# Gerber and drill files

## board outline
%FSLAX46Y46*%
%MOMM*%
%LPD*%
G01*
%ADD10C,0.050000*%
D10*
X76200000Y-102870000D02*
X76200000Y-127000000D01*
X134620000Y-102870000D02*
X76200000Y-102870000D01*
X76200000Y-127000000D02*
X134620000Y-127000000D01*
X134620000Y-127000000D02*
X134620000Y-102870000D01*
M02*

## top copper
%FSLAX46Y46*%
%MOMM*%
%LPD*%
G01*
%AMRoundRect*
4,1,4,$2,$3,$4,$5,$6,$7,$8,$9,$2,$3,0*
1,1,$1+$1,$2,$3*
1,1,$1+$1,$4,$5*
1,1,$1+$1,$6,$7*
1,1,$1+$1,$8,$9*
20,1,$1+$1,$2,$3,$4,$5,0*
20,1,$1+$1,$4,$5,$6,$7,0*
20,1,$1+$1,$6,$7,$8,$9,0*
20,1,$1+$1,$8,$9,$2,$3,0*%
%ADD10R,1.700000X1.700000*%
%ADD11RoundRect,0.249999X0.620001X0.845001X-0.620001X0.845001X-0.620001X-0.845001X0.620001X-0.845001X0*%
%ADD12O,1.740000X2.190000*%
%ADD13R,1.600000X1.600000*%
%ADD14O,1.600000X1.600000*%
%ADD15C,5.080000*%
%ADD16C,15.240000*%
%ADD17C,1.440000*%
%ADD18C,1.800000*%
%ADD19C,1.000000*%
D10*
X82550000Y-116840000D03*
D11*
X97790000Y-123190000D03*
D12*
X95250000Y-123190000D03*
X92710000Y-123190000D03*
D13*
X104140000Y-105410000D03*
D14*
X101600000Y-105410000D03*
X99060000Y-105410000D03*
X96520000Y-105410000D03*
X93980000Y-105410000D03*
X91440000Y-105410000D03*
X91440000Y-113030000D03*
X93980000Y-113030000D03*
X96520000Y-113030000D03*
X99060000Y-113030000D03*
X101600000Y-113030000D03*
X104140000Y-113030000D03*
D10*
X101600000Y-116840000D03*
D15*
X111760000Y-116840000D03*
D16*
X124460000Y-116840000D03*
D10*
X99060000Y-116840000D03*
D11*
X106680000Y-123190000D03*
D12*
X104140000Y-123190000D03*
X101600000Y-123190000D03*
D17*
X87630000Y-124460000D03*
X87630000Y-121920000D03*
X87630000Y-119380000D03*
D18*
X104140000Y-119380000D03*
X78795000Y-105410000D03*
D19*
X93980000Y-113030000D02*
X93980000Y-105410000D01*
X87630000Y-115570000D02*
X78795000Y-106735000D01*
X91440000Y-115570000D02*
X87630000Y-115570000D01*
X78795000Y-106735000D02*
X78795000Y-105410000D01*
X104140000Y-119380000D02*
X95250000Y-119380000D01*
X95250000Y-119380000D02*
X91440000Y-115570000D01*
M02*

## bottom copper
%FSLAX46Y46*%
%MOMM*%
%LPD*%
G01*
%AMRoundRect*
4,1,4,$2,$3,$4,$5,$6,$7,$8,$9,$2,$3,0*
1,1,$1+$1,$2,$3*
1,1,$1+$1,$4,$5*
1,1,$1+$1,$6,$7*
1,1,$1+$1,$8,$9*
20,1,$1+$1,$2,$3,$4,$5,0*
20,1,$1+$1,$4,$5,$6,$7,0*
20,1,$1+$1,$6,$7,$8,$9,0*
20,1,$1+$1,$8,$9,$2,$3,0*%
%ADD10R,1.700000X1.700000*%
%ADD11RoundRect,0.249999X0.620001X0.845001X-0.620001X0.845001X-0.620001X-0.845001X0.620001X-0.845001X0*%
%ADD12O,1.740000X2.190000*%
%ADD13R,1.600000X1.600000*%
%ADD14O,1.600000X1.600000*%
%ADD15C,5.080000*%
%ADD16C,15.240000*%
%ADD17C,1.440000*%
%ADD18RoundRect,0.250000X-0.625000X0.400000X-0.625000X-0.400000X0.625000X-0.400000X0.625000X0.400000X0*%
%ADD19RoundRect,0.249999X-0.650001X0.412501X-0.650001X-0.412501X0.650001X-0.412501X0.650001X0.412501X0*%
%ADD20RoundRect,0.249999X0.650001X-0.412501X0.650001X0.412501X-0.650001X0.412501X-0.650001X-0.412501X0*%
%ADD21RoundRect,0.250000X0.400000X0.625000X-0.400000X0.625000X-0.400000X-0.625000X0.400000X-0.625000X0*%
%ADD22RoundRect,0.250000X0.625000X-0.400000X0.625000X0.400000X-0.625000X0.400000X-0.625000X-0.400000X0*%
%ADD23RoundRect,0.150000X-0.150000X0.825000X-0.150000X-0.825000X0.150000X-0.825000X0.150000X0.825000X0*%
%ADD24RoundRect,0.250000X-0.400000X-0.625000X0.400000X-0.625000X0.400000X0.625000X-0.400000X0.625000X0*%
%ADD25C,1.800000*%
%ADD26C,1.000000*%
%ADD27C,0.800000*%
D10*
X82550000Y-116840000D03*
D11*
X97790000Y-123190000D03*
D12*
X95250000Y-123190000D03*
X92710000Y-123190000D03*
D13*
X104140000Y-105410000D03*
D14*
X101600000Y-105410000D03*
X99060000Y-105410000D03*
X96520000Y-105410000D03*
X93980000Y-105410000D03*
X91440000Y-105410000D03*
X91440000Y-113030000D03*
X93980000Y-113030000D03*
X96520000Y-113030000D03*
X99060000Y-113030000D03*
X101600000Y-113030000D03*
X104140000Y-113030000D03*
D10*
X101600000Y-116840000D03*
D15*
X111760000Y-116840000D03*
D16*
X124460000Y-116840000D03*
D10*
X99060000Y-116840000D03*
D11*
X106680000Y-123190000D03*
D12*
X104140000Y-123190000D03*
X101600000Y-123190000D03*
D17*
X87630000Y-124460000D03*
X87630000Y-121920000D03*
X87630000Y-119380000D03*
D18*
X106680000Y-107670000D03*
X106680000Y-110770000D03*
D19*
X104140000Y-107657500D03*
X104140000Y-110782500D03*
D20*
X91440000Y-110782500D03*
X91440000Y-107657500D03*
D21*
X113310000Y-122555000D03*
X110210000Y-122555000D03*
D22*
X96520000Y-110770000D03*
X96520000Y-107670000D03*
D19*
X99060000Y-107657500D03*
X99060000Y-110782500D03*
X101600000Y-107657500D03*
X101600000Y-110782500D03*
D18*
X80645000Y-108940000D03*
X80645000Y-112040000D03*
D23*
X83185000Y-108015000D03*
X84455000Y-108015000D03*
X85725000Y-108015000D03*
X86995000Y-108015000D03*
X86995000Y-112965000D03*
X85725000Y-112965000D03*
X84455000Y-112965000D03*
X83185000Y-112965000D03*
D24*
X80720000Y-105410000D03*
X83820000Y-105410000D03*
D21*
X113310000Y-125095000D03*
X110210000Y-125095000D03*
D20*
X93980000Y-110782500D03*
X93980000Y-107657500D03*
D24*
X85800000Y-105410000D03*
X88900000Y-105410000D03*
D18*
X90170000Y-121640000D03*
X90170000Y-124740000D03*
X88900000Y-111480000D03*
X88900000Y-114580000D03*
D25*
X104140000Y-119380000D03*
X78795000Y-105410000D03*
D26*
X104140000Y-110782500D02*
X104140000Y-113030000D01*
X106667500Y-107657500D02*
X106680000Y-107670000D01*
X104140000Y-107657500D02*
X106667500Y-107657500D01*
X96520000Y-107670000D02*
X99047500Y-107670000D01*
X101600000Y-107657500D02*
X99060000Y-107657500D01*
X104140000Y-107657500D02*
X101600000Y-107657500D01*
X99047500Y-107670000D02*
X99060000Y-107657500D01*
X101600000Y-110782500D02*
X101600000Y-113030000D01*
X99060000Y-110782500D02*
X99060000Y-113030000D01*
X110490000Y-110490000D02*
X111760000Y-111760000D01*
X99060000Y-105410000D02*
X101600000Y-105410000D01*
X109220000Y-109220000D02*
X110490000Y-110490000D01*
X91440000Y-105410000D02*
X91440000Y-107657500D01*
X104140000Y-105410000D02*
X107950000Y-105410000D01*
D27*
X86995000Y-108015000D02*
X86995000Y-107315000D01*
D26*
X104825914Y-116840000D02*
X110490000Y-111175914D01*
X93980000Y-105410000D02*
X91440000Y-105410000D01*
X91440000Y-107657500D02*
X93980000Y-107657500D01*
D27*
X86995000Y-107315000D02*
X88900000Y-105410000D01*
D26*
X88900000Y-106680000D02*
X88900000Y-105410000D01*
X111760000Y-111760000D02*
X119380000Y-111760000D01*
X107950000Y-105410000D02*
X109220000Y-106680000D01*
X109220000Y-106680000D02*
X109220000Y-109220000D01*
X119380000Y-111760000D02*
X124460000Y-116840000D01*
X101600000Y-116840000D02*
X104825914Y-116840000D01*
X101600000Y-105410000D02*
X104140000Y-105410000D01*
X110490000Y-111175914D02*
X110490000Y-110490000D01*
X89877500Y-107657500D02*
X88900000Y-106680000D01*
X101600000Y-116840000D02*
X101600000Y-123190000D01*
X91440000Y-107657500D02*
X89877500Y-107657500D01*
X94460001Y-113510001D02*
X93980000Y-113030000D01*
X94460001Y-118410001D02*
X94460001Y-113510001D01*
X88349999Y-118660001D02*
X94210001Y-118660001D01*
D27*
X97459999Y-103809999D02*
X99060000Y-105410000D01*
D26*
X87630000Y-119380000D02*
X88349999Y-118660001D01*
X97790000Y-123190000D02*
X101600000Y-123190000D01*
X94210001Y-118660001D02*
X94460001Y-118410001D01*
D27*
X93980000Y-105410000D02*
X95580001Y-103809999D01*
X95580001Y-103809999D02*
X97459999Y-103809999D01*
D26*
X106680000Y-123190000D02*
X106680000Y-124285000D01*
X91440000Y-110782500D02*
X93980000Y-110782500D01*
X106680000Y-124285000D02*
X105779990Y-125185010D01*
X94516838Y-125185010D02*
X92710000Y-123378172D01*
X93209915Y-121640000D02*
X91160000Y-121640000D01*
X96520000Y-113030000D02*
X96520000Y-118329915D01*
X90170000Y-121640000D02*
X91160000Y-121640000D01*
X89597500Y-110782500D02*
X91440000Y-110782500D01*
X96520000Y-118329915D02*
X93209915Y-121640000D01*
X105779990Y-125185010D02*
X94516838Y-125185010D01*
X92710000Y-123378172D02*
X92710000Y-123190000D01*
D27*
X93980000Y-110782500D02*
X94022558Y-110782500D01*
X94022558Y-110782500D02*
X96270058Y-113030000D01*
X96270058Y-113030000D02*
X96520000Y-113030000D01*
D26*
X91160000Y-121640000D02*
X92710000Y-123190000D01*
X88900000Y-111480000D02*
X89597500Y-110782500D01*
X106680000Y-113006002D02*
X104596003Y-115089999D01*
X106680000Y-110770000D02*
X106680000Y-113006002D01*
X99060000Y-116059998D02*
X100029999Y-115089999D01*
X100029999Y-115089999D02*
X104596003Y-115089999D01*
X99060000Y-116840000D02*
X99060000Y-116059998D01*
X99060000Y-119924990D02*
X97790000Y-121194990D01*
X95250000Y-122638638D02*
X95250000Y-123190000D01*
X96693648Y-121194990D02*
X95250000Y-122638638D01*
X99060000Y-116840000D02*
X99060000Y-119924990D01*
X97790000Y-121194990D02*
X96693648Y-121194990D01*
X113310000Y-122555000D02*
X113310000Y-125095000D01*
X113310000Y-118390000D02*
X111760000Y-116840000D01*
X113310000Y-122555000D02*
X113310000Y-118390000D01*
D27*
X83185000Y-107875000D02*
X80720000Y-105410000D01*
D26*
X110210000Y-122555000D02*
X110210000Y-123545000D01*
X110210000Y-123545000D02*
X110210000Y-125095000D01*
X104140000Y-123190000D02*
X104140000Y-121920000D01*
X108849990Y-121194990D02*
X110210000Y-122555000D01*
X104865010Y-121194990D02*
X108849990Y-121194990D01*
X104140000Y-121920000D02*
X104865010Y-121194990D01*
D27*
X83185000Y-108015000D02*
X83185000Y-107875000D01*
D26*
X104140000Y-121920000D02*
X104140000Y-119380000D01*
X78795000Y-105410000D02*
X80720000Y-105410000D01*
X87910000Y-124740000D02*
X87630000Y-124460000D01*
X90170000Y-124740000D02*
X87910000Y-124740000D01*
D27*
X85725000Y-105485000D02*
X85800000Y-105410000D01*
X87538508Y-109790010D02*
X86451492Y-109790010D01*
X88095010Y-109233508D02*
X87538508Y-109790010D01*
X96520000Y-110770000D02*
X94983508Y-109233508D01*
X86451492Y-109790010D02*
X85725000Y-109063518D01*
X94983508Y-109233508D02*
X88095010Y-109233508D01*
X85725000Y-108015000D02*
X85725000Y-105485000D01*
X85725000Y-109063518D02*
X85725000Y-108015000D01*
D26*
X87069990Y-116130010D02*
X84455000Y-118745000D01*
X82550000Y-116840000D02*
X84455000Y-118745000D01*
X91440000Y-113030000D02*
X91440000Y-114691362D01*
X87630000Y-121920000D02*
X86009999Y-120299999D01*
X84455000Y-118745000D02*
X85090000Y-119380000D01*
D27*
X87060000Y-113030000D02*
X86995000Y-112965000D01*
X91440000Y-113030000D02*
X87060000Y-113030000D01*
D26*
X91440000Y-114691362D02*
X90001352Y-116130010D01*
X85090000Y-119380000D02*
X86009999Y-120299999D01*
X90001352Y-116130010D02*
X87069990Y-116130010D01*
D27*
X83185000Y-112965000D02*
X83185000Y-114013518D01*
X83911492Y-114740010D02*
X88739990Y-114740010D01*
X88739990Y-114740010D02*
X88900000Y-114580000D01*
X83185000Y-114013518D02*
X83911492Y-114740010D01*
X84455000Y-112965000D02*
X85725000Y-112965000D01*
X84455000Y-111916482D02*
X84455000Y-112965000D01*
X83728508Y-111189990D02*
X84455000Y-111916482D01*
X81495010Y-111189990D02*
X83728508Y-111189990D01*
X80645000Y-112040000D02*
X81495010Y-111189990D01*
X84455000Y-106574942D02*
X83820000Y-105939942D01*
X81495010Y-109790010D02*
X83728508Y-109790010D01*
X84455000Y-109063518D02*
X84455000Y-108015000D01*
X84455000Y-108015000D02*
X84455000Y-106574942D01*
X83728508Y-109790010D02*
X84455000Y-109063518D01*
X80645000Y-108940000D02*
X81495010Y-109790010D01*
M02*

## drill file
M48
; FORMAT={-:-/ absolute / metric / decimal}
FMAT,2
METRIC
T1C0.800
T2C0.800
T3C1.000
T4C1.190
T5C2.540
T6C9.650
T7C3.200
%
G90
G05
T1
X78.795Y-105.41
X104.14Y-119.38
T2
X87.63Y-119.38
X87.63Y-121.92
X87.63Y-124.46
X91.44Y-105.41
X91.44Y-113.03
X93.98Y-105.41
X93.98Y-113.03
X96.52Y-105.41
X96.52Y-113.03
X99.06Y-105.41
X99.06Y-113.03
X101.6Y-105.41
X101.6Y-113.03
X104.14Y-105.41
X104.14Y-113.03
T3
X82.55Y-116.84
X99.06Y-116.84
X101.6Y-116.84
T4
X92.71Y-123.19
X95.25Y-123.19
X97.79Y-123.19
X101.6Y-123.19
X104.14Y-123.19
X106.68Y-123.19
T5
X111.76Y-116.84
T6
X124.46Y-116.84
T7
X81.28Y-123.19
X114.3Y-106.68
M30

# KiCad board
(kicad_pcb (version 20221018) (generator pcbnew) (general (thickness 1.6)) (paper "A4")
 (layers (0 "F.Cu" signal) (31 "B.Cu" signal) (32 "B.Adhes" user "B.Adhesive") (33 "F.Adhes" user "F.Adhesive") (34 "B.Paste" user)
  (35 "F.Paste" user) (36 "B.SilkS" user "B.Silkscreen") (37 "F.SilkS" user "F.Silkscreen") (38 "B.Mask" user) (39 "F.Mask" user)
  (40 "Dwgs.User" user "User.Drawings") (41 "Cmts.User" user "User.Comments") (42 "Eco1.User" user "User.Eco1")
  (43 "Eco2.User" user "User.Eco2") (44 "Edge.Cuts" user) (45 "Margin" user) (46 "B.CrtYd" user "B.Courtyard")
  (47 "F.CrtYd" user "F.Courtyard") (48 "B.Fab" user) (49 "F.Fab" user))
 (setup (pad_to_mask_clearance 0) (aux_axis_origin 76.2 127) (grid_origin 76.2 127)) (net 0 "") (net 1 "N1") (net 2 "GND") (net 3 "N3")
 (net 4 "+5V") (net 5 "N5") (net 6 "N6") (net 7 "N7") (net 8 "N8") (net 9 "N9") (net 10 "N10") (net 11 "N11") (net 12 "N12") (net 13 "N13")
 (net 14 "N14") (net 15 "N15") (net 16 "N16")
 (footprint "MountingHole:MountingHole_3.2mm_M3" (layer "F.Cu") (at 114.3 106.68)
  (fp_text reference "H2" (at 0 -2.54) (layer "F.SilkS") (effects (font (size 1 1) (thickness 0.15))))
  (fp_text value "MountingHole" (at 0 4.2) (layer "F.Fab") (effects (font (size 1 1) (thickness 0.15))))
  (pad "" np_thru_hole circle (at 0 0) (size 3.2 3.2) (drill 3.2) (layers "*.Cu" "*.Mask")))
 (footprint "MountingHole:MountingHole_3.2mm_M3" (layer "F.Cu") (at 81.28 123.19)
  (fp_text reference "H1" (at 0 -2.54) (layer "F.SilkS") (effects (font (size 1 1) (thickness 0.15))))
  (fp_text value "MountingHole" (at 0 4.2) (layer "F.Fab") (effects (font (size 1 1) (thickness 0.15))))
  (pad "" np_thru_hole circle (at 0 0) (size 3.2 3.2) (drill 3.2) (layers "*.Cu" "*.Mask")))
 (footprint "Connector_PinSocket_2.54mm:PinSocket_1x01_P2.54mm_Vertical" (layer "F.Cu") (at 82.55 116.84)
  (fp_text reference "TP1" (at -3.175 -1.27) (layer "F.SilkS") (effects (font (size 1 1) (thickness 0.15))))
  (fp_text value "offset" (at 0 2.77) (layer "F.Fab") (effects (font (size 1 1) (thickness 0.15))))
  (pad "1" thru_hole rect (at 0 0) (size 1.7 1.7) (drill 1) (layers "*.Cu" "*.Mask") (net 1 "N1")))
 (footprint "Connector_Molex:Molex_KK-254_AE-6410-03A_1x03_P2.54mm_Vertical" (layer "F.Cu") (at 97.79 123.19 180)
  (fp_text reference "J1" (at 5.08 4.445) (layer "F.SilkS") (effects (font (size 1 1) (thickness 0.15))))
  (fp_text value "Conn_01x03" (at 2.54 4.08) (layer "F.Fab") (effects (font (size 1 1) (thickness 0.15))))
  (pad "1" thru_hole roundrect (at 0 0 180) (size 1.74 2.19) (drill 1.19) (layers "*.Cu" "*.Mask") (roundrect_rratio 0.1436775862)
   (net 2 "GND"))
  (pad "2" thru_hole oval (at 2.54 0 180) (size 1.74 2.19) (drill 1.19) (layers "*.Cu" "*.Mask") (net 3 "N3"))
  (pad "3" thru_hole oval (at 5.08 0 180) (size 1.74 2.19) (drill 1.19) (layers "*.Cu" "*.Mask") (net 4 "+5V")))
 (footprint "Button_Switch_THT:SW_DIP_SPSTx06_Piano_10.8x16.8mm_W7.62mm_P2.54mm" (layer "F.Cu") (at 104.14 105.41 -90)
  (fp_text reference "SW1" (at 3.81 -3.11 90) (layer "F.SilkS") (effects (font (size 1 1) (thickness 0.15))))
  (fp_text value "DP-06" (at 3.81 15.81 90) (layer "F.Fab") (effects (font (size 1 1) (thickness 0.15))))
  (pad "1" thru_hole rect (at 0 0 270) (size 1.6 1.6) (drill 0.8) (layers "*.Cu" "*.Mask") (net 2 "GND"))
  (pad "2" thru_hole oval (at 0 2.54 270) (size 1.6 1.6) (drill 0.8) (layers "*.Cu" "*.Mask") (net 2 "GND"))
  (pad "3" thru_hole oval (at 0 5.08 270) (size 1.6 1.6) (drill 0.8) (layers "*.Cu" "*.Mask") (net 2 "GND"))
  (pad "4" thru_hole oval (at 0 7.62 270) (size 1.6 1.6) (drill 0.8) (layers "*.Cu" "*.Mask") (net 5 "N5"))
  (pad "5" thru_hole oval (at 0 10.16 270) (size 1.6 1.6) (drill 0.8) (layers "*.Cu" "*.Mask") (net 2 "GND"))
  (pad "6" thru_hole oval (at 0 12.7 270) (size 1.6 1.6) (drill 0.8) (layers "*.Cu" "*.Mask") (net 2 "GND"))
  (pad "7" thru_hole oval (at 7.62 12.7 270) (size 1.6 1.6) (drill 0.8) (layers "*.Cu" "*.Mask") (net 1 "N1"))
  (pad "8" thru_hole oval (at 7.62 10.16 270) (size 1.6 1.6) (drill 0.8) (layers "*.Cu" "*.Mask") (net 2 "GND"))
  (pad "9" thru_hole oval (at 7.62 7.62 270) (size 1.6 1.6) (drill 0.8) (layers "*.Cu" "*.Mask") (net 4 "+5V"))
  (pad "10" thru_hole oval (at 7.62 5.08 270) (size 1.6 1.6) (drill 0.8) (layers "*.Cu" "*.Mask") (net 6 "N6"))
  (pad "11" thru_hole oval (at 7.62 2.54 270) (size 1.6 1.6) (drill 0.8) (layers "*.Cu" "*.Mask") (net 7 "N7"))
  (pad "12" thru_hole oval (at 7.62 0 270) (size 1.6 1.6) (drill 0.8) (layers "*.Cu" "*.Mask") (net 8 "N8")))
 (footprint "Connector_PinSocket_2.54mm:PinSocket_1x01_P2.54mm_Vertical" (layer "F.Cu") (at 101.6 116.84)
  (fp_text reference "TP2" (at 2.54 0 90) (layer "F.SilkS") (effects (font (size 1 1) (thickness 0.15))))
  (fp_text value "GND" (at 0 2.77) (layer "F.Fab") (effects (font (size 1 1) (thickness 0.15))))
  (pad "1" thru_hole rect (at 0 0) (size 1.7 1.7) (drill 1) (layers "*.Cu" "*.Mask") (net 2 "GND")))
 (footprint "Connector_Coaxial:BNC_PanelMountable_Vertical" (layer "F.Cu") (at 111.76 116.84 180)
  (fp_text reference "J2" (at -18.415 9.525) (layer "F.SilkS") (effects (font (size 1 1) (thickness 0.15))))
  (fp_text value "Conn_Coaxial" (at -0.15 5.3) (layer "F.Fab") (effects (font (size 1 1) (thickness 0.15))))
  (pad "1" thru_hole circle (at 0 0 180) (size 5.08 5.08) (drill 2.54) (layers "*.Cu" "*.Mask") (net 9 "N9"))
  (pad "2" thru_hole circle (at -12.7 0 180) (size 15.24 15.24) (drill 9.65) (layers "*.Cu" "*.Mask") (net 2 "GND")))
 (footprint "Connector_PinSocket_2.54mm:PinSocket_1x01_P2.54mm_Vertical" (layer "F.Cu") (at 99.06 116.84)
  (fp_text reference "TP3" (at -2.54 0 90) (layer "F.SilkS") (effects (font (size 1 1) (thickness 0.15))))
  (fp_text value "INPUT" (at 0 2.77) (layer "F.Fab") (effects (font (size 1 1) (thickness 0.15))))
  (pad "1" thru_hole rect (at 0 0) (size 1.7 1.7) (drill 1) (layers "*.Cu" "*.Mask") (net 3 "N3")))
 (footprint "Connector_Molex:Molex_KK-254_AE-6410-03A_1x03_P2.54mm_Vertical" (layer "F.Cu") (at 106.68 123.19 180)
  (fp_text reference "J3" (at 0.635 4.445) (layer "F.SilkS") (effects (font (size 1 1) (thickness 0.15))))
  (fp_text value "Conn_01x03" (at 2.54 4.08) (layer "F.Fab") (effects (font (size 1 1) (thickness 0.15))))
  (pad "1" thru_hole roundrect (at 0 0 180) (size 1.74 2.19) (drill 1.19) (layers "*.Cu" "*.Mask") (roundrect_rratio 0.1436775862)
   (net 4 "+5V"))
  (pad "2" thru_hole oval (at 2.54 0 180) (size 1.74 2.19) (drill 1.19) (layers "*.Cu" "*.Mask") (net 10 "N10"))
  (pad "3" thru_hole oval (at 5.08 0 180) (size 1.74 2.19) (drill 1.19) (layers "*.Cu" "*.Mask") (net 2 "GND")))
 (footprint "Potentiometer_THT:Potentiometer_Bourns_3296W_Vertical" (layer "F.Cu") (at 87.63 124.46 -90)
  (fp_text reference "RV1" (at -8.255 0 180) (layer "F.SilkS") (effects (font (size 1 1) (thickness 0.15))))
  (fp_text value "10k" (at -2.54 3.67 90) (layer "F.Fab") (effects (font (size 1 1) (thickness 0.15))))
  (pad "1" thru_hole circle (at 0 0 270) (size 1.44 1.44) (drill 0.8) (layers "*.Cu" "*.Mask") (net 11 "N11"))
  (pad "2" thru_hole circle (at -2.54 0 270) (size 1.44 1.44) (drill 0.8) (layers "*.Cu" "*.Mask") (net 1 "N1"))
  (pad "3" thru_hole circle (at -5.08 0 270) (size 1.44 1.44) (drill 0.8) (layers "*.Cu" "*.Mask") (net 2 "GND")))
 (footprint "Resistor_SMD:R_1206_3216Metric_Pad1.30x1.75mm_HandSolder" (layer "B.Cu") (at 106.68 109.22 -90)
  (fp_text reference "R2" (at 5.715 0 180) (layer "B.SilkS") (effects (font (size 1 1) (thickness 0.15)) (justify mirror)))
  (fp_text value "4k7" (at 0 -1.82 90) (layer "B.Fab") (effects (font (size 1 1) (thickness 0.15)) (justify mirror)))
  (pad "1" smd roundrect (at -1.55 0 270) (size 1.3 1.75) (layers "B.Cu" "B.Paste" "B.Mask") (roundrect_rratio 0.1923076923) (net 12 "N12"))
  (pad "2" smd roundrect (at 1.55 0 270) (size 1.3 1.75) (layers "B.Cu" "B.Paste" "B.Mask") (roundrect_rratio 0.1923076923) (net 3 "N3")))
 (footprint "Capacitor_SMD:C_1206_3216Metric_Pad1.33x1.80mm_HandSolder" (layer "B.Cu") (at 104.14 109.22 -90)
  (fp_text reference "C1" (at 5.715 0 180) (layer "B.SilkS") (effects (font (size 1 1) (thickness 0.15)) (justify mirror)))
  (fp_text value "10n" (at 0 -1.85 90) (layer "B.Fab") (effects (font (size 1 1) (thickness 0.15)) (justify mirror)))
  (pad "1" smd roundrect (at -1.5625 0 270) (size 1.325 1.8) (layers "B.Cu" "B.Paste" "B.Mask") (roundrect_rratio 0.1886784906)
   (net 12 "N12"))
  (pad "2" smd roundrect (at 1.5625 0 270) (size 1.325 1.8) (layers "B.Cu" "B.Paste" "B.Mask") (roundrect_rratio 0.1886784906) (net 8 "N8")))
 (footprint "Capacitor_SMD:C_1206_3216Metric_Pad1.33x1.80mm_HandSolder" (layer "B.Cu") (at 91.44 109.22 90)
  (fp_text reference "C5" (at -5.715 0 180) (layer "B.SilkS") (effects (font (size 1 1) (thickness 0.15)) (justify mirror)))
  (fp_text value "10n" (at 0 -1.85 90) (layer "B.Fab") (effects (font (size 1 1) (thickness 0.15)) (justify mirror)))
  (pad "1" smd roundrect (at -1.5625 0 90) (size 1.325 1.8) (layers "B.Cu" "B.Paste" "B.Mask") (roundrect_rratio 0.1886784906) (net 4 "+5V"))
  (pad "2" smd roundrect (at 1.5625 0 90) (size 1.325 1.8) (layers "B.Cu" "B.Paste" "B.Mask") (roundrect_rratio 0.1886784906) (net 2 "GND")))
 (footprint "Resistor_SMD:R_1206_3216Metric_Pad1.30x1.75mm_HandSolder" (layer "B.Cu") (at 111.76 122.555 180)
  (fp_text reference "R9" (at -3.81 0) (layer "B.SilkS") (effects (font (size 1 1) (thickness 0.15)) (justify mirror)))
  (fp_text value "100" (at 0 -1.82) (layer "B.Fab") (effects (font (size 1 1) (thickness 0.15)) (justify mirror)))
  (pad "1" smd roundrect (at -1.55 0 180) (size 1.3 1.75) (layers "B.Cu" "B.Paste" "B.Mask") (roundrect_rratio 0.1923076923) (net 9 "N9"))
  (pad "2" smd roundrect (at 1.55 0 180) (size 1.3 1.75) (layers "B.Cu" "B.Paste" "B.Mask") (roundrect_rratio 0.1923076923) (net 10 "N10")))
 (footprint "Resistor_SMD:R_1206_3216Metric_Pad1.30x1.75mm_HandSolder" (layer "B.Cu") (at 96.52 109.22 90)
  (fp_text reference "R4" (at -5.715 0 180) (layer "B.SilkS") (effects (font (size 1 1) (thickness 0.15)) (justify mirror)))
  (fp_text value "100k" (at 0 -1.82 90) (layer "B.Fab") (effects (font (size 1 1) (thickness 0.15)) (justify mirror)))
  (pad "1" smd roundrect (at -1.55 0 90) (size 1.3 1.75) (layers "B.Cu" "B.Paste" "B.Mask") (roundrect_rratio 0.1923076923) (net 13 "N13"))
  (pad "2" smd roundrect (at 1.55 0 90) (size 1.3 1.75) (layers "B.Cu" "B.Paste" "B.Mask") (roundrect_rratio 0.1923076923) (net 12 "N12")))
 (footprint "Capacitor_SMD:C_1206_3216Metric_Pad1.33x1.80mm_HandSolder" (layer "B.Cu") (at 99.06 109.22 -90)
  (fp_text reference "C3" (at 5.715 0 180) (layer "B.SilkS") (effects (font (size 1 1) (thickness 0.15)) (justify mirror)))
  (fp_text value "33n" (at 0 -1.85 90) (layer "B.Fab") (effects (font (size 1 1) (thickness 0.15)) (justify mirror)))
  (pad "1" smd roundrect (at -1.5625 0 270) (size 1.325 1.8) (layers "B.Cu" "B.Paste" "B.Mask") (roundrect_rratio 0.1886784906)
   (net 12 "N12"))
  (pad "2" smd roundrect (at 1.5625 0 270) (size 1.325 1.8) (layers "B.Cu" "B.Paste" "B.Mask") (roundrect_rratio 0.1886784906) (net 6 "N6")))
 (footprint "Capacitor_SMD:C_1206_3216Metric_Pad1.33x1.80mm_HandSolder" (layer "B.Cu") (at 101.6 109.22 -90)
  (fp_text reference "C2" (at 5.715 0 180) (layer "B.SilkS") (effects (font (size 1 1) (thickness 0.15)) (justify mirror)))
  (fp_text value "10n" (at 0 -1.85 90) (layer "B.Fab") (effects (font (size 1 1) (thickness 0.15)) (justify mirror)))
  (pad "1" smd roundrect (at -1.5625 0 270) (size 1.325 1.8) (layers "B.Cu" "B.Paste" "B.Mask") (roundrect_rratio 0.1886784906)
   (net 12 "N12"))
  (pad "2" smd roundrect (at 1.5625 0 270) (size 1.325 1.8) (layers "B.Cu" "B.Paste" "B.Mask") (roundrect_rratio 0.1886784906) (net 7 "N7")))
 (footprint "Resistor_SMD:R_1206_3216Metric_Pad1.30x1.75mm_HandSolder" (layer "B.Cu") (at 80.645 110.49 -90)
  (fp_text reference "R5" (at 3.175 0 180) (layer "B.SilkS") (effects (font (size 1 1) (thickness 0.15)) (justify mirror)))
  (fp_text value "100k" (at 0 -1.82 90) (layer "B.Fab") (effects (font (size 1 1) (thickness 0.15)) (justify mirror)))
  (pad "1" smd roundrect (at -1.55 0 270) (size 1.3 1.75) (layers "B.Cu" "B.Paste" "B.Mask") (roundrect_rratio 0.1923076923) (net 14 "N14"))
  (pad "2" smd roundrect (at 1.55 0 270) (size 1.3 1.75) (layers "B.Cu" "B.Paste" "B.Mask") (roundrect_rratio 0.1923076923) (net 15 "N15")))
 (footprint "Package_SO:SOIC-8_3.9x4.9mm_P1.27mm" (layer "B.Cu") (at 85.09 110.49 -90)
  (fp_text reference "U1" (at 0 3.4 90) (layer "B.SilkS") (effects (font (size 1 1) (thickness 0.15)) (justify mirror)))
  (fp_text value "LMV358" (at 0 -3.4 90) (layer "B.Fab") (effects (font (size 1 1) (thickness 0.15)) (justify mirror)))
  (pad "1" smd roundrect (at -2.475 1.905 270) (size 1.95 0.6) (layers "B.Cu" "B.Paste" "B.Mask") (roundrect_rratio 0.25) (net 10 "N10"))
  (pad "2" smd roundrect (at -2.475 0.635 270) (size 1.95 0.6) (layers "B.Cu" "B.Paste" "B.Mask") (roundrect_rratio 0.25) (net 14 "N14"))
  (pad "3" smd roundrect (at -2.475 -0.635 270) (size 1.95 0.6) (layers "B.Cu" "B.Paste" "B.Mask") (roundrect_rratio 0.25) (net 13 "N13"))
  (pad "4" smd roundrect (at -2.475 -1.905 270) (size 1.95 0.6) (layers "B.Cu" "B.Paste" "B.Mask") (roundrect_rratio 0.25) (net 2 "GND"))
  (pad "5" smd roundrect (at 2.475 -1.905 270) (size 1.95 0.6) (layers "B.Cu" "B.Paste" "B.Mask") (roundrect_rratio 0.25) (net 1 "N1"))
  (pad "6" smd roundrect (at 2.475 -0.635 270) (size 1.95 0.6) (layers "B.Cu" "B.Paste" "B.Mask") (roundrect_rratio 0.25) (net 15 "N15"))
  (pad "7" smd roundrect (at 2.475 0.635 270) (size 1.95 0.6) (layers "B.Cu" "B.Paste" "B.Mask") (roundrect_rratio 0.25) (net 15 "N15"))
  (pad "8" smd roundrect (at 2.475 1.905 270) (size 1.95 0.6) (layers "B.Cu" "B.Paste" "B.Mask") (roundrect_rratio 0.25) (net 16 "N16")))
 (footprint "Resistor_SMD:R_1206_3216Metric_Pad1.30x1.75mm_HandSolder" (layer "B.Cu") (at 82.27 105.41)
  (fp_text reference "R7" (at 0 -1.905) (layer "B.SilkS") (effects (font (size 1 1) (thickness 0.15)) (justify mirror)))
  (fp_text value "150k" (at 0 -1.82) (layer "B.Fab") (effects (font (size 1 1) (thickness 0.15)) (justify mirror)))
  (pad "1" smd roundrect (at -1.55 0) (size 1.3 1.75) (layers "B.Cu" "B.Paste" "B.Mask") (roundrect_rratio 0.1923076923) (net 10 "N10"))
  (pad "2" smd roundrect (at 1.55 0) (size 1.3 1.75) (layers "B.Cu" "B.Paste" "B.Mask") (roundrect_rratio 0.1923076923) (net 14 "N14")))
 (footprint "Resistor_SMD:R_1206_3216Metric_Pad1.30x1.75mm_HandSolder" (layer "B.Cu") (at 111.76 125.095 180)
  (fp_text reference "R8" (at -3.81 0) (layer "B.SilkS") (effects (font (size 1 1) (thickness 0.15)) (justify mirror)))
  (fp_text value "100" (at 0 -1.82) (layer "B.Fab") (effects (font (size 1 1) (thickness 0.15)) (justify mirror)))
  (pad "1" smd roundrect (at -1.55 0 180) (size 1.3 1.75) (layers "B.Cu" "B.Paste" "B.Mask") (roundrect_rratio 0.1923076923) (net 9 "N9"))
  (pad "2" smd roundrect (at 1.55 0 180) (size 1.3 1.75) (layers "B.Cu" "B.Paste" "B.Mask") (roundrect_rratio 0.1923076923) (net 10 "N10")))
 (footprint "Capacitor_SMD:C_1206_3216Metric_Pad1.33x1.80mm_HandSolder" (layer "B.Cu") (at 93.98 109.22 90)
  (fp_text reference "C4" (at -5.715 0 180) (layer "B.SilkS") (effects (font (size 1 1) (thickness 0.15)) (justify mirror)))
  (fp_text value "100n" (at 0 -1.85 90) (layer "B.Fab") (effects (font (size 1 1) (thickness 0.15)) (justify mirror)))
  (pad "1" smd roundrect (at -1.5625 0 90) (size 1.325 1.8) (layers "B.Cu" "B.Paste" "B.Mask") (roundrect_rratio 0.1886784906) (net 4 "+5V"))
  (pad "2" smd roundrect (at 1.5625 0 90) (size 1.325 1.8) (layers "B.Cu" "B.Paste" "B.Mask") (roundrect_rratio 0.1886784906) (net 2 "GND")))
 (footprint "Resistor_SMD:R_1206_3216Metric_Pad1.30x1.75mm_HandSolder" (layer "B.Cu") (at 87.35 105.41)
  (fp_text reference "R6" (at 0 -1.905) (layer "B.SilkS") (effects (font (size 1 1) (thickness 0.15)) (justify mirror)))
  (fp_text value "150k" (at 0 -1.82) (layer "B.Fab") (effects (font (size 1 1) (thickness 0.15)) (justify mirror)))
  (pad "1" smd roundrect (at -1.55 0) (size 1.3 1.75) (layers "B.Cu" "B.Paste" "B.Mask") (roundrect_rratio 0.1923076923) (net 13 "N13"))
  (pad "2" smd roundrect (at 1.55 0) (size 1.3 1.75) (layers "B.Cu" "B.Paste" "B.Mask") (roundrect_rratio 0.1923076923) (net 2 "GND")))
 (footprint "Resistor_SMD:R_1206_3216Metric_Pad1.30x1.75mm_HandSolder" (layer "B.Cu") (at 90.17 123.19 -90)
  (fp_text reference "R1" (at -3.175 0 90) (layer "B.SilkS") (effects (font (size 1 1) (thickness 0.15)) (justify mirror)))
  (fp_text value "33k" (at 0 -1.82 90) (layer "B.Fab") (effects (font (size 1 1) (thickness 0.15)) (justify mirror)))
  (pad "1" smd roundrect (at -1.55 0 270) (size 1.3 1.75) (layers "B.Cu" "B.Paste" "B.Mask") (roundrect_rratio 0.1923076923) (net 4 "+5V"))
  (pad "2" smd roundrect (at 1.55 0 270) (size 1.3 1.75) (layers "B.Cu" "B.Paste" "B.Mask") (roundrect_rratio 0.1923076923) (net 11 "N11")))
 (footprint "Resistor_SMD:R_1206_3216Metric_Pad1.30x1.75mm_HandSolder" (layer "B.Cu") (at 88.9 113.03 -90)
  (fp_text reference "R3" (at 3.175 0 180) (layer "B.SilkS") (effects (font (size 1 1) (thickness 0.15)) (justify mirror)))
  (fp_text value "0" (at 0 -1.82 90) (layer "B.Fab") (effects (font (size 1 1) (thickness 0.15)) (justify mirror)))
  (pad "1" smd roundrect (at -1.55 0 270) (size 1.3 1.75) (layers "B.Cu" "B.Paste" "B.Mask") (roundrect_rratio 0.1923076923) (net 4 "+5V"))
  (pad "2" smd roundrect (at 1.55 0 270) (size 1.3 1.75) (layers "B.Cu" "B.Paste" "B.Mask") (roundrect_rratio 0.1923076923) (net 16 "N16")))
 (gr_line (start 76.2 102.87) (end 76.2 127) (stroke (width 0.05) (type solid)) (layer "Edge.Cuts"))
 (gr_line (start 134.62 102.87) (end 76.2 102.87) (stroke (width 0.05) (type solid)) (layer "Edge.Cuts"))
 (gr_line (start 76.2 127) (end 134.62 127) (stroke (width 0.05) (type solid)) (layer "Edge.Cuts"))
 (gr_line (start 134.62 127) (end 134.62 102.87) (stroke (width 0.05) (type solid)) (layer "Edge.Cuts"))
 (segment (start 104.14 110.7825) (end 104.14 113.03) (width 1) (layer "B.Cu") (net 8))
 (segment (start 106.6675 107.6575) (end 106.68 107.67) (width 1) (layer "B.Cu") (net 12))
 (segment (start 104.14 107.6575) (end 106.6675 107.6575) (width 1) (layer "B.Cu") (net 12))
 (segment (start 96.52 107.67) (end 99.0475 107.67) (width 1) (layer "B.Cu") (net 12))
 (segment (start 101.6 107.6575) (end 99.06 107.6575) (width 1) (layer "B.Cu") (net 12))
 (segment (start 104.14 107.6575) (end 101.6 107.6575) (width 1) (layer "B.Cu") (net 12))
 (segment (start 99.0475 107.67) (end 99.06 107.6575) (width 1) (layer "B.Cu") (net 12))
 (segment (start 101.6 110.7825) (end 101.6 113.03) (width 1) (layer "B.Cu") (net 7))
 (segment (start 99.06 110.7825) (end 99.06 113.03) (width 1) (layer "B.Cu") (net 6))
 (segment (start 93.98 113.03) (end 93.98 105.41) (width 1) (layer "F.Cu") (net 2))
 (segment (start 110.49 110.49) (end 111.76 111.76) (width 1) (layer "B.Cu") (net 2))
 (segment (start 99.06 105.41) (end 101.6 105.41) (width 1) (layer "B.Cu") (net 2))
 (segment (start 109.22 109.22) (end 110.49 110.49) (width 1) (layer "B.Cu") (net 2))
 (segment (start 91.44 105.41) (end 91.44 107.6575) (width 1) (layer "B.Cu") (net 2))
 (segment (start 104.14 105.41) (end 107.95 105.41) (width 1) (layer "B.Cu") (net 2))
 (segment (start 86.995 108.015) (end 86.995 107.315) (width 0.8) (layer "B.Cu") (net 2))
 (segment (start 104.825914 116.84) (end 110.49 111.175914) (width 1) (layer "B.Cu") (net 2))
 (segment (start 93.98 105.41) (end 91.44 105.41) (width 1) (layer "B.Cu") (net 2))
 (segment (start 91.44 107.6575) (end 93.98 107.6575) (width 1) (layer "B.Cu") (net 2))
 (segment (start 86.995 107.315) (end 88.9 105.41) (width 0.8) (layer "B.Cu") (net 2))
 (segment (start 88.9 106.68) (end 88.9 105.41) (width 1) (layer "B.Cu") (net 2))
 (segment (start 111.76 111.76) (end 119.38 111.76) (width 1) (layer "B.Cu") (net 2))
 (segment (start 107.95 105.41) (end 109.22 106.68) (width 1) (layer "B.Cu") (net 2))
 (segment (start 109.22 106.68) (end 109.22 109.22) (width 1) (layer "B.Cu") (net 2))
 (segment (start 119.38 111.76) (end 124.46 116.84) (width 1) (layer "B.Cu") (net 2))
 (segment (start 101.6 116.84) (end 104.825914 116.84) (width 1) (layer "B.Cu") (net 2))
 (segment (start 101.6 105.41) (end 104.14 105.41) (width 1) (layer "B.Cu") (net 2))
 (segment (start 110.49 111.175914) (end 110.49 110.49) (width 1) (layer "B.Cu") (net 2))
 (segment (start 89.8775 107.6575) (end 88.9 106.68) (width 1) (layer "B.Cu") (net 2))
 (segment (start 101.6 116.84) (end 101.6 123.19) (width 1) (layer "B.Cu") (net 2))
 (segment (start 91.44 107.6575) (end 89.8775 107.6575) (width 1) (layer "B.Cu") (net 2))
 (segment (start 94.460001 113.510001) (end 93.98 113.03) (width 1) (layer "B.Cu") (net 2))
 (segment (start 94.460001 118.410001) (end 94.460001 113.510001) (width 1) (layer "B.Cu") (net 2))
 (segment (start 88.349999 118.660001) (end 94.210001 118.660001) (width 1) (layer "B.Cu") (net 2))
 (segment (start 97.459999 103.809999) (end 99.06 105.41) (width 0.8) (layer "B.Cu") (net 2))
 (segment (start 87.63 119.38) (end 88.349999 118.660001) (width 1) (layer "B.Cu") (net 2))
 (segment (start 97.79 123.19) (end 101.6 123.19) (width 1) (layer "B.Cu") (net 2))
 (segment (start 94.210001 118.660001) (end 94.460001 118.410001) (width 1) (layer "B.Cu") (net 2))
 (segment (start 93.98 105.41) (end 95.580001 103.809999) (width 0.8) (layer "B.Cu") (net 2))
 (segment (start 95.580001 103.809999) (end 97.459999 103.809999) (width 0.8) (layer "B.Cu") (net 2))
 (segment (start 106.68 123.19) (end 106.68 124.285) (width 1) (layer "B.Cu") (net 4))
 (segment (start 91.44 110.7825) (end 93.98 110.7825) (width 1) (layer "B.Cu") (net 4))
 (segment (start 106.68 124.285) (end 105.77999 125.18501) (width 1) (layer "B.Cu") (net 4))
 (segment (start 94.516838 125.18501) (end 92.71 123.378172) (width 1) (layer "B.Cu") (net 4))
 (segment (start 93.209915 121.64) (end 91.16 121.64) (width 1) (layer "B.Cu") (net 4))
 (segment (start 96.52 113.03) (end 96.52 118.329915) (width 1) (layer "B.Cu") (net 4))
 (segment (start 90.17 121.64) (end 91.16 121.64) (width 1) (layer "B.Cu") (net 4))
 (segment (start 89.5975 110.7825) (end 91.44 110.7825) (width 1) (layer "B.Cu") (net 4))
 (segment (start 96.52 118.329915) (end 93.209915 121.64) (width 1) (layer "B.Cu") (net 4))
 (segment (start 105.77999 125.18501) (end 94.516838 125.18501) (width 1) (layer "B.Cu") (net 4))
 (segment (start 92.71 123.378172) (end 92.71 123.19) (width 1) (layer "B.Cu") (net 4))
 (segment (start 93.98 110.7825) (end 94.022558 110.7825) (width 0.8) (layer "B.Cu") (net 4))
 (segment (start 94.022558 110.7825) (end 96.270058 113.03) (width 0.8) (layer "B.Cu") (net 4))
 (segment (start 96.270058 113.03) (end 96.52 113.03) (width 0.8) (layer "B.Cu") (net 4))
 (segment (start 91.16 121.64) (end 92.71 123.19) (width 1) (layer "B.Cu") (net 4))
 (segment (start 88.9 111.48) (end 89.5975 110.7825) (width 1) (layer "B.Cu") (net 4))
 (segment (start 106.68 113.006002) (end 104.596003 115.089999) (width 1) (layer "B.Cu") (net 3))
 (segment (start 106.68 110.77) (end 106.68 113.006002) (width 1) (layer "B.Cu") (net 3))
 (segment (start 99.06 116.059998) (end 100.029999 115.089999) (width 1) (layer "B.Cu") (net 3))
 (segment (start 100.029999 115.089999) (end 104.596003 115.089999) (width 1) (layer "B.Cu") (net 3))
 (segment (start 99.06 116.84) (end 99.06 116.059998) (width 1) (layer "B.Cu") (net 3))
 (segment (start 99.06 119.92499) (end 97.79 121.19499) (width 1) (layer "B.Cu") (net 3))
 (segment (start 95.25 122.638638) (end 95.25 123.19) (width 1) (layer "B.Cu") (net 3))
 (segment (start 96.693648 121.19499) (end 95.25 122.638638) (width 1) (layer "B.Cu") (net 3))
 (segment (start 99.06 116.84) (end 99.06 119.92499) (width 1) (layer "B.Cu") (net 3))
 (segment (start 97.79 121.19499) (end 96.693648 121.19499) (width 1) (layer "B.Cu") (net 3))
 (segment (start 113.31 122.555) (end 113.31 125.095) (width 1) (layer "B.Cu") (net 9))
 (segment (start 113.31 118.39) (end 111.76 116.84) (width 1) (layer "B.Cu") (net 9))
 (segment (start 113.31 122.555) (end 113.31 118.39) (width 1) (layer "B.Cu") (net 9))
 (segment (start 87.63 115.57) (end 78.795 106.735) (width 1) (layer "F.Cu") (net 10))
 (segment (start 91.44 115.57) (end 87.63 115.57) (width 1) (layer "F.Cu") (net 10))
 (segment (start 78.795 106.735) (end 78.795 105.41) (width 1) (layer "F.Cu") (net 10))
 (segment (start 104.14 119.38) (end 95.25 119.38) (width 1) (layer "F.Cu") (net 10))
 (segment (start 95.25 119.38) (end 91.44 115.57) (width 1) (layer "F.Cu") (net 10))
 (via (at 104.14 119.38) (size 1.8) (drill 0.8) (layers "F.Cu" "B.Cu") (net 10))
 (via (at 78.795 105.41) (size 1.8) (drill 0.8) (layers "F.Cu" "B.Cu") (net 10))
 (segment (start 83.185 107.875) (end 80.72 105.41) (width 0.8) (layer "B.Cu") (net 10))
 (segment (start 110.21 122.555) (end 110.21 123.545) (width 1) (layer "B.Cu") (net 10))
 (segment (start 110.21 123.545) (end 110.21 125.095) (width 1) (layer "B.Cu") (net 10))
 (segment (start 104.14 123.19) (end 104.14 121.92) (width 1) (layer "B.Cu") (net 10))
 (segment (start 108.84999 121.19499) (end 110.21 122.555) (width 1) (layer "B.Cu") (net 10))
 (segment (start 104.86501 121.19499) (end 108.84999 121.19499) (width 1) (layer "B.Cu") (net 10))
 (segment (start 104.14 121.92) (end 104.86501 121.19499) (width 1) (layer "B.Cu") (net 10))
 (segment (start 83.185 108.015) (end 83.185 107.875) (width 0.8) (layer "B.Cu") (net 10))
 (segment (start 104.14 121.92) (end 104.14 119.38) (width 1) (layer "B.Cu") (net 10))
 (segment (start 78.795 105.41) (end 80.72 105.41) (width 1) (layer "B.Cu") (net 10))
 (segment (start 87.91 124.74) (end 87.63 124.46) (width 1) (layer "B.Cu") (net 11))
 (segment (start 90.17 124.74) (end 87.91 124.74) (width 1) (layer "B.Cu") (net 11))
 (segment (start 85.725 105.485) (end 85.8 105.41) (width 0.8) (layer "B.Cu") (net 13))
 (segment (start 87.538508 109.79001) (end 86.451492 109.79001) (width 0.8) (layer "B.Cu") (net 13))
 (segment (start 88.09501 109.233508) (end 87.538508 109.79001) (width 0.8) (layer "B.Cu") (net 13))
 (segment (start 96.52 110.77) (end 94.983508 109.233508) (width 0.8) (layer "B.Cu") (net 13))
 (segment (start 86.451492 109.79001) (end 85.725 109.063518) (width 0.8) (layer "B.Cu") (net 13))
 (segment (start 94.983508 109.233508) (end 88.09501 109.233508) (width 0.8) (layer "B.Cu") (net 13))
 (segment (start 85.725 108.015) (end 85.725 105.485) (width 0.8) (layer "B.Cu") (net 13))
 (segment (start 85.725 109.063518) (end 85.725 108.015) (width 0.8) (layer "B.Cu") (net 13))
 (segment (start 87.06999 116.13001) (end 84.455 118.745) (width 1) (layer "B.Cu") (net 1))
 (segment (start 82.55 116.84) (end 84.455 118.745) (width 1) (layer "B.Cu") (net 1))
 (segment (start 91.44 113.03) (end 91.44 114.691362) (width 1) (layer "B.Cu") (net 1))
 (segment (start 87.63 121.92) (end 86.009999 120.299999) (width 1) (layer "B.Cu") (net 1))
 (segment (start 84.455 118.745) (end 85.09 119.38) (width 1) (layer "B.Cu") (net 1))
 (segment (start 87.06 113.03) (end 86.995 112.965) (width 0.8) (layer "B.Cu") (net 1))
 (segment (start 91.44 113.03) (end 87.06 113.03) (width 0.8) (layer "B.Cu") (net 1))
 (segment (start 91.44 114.691362) (end 90.001352 116.13001) (width 1) (layer "B.Cu") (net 1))
 (segment (start 85.09 119.38) (end 86.009999 120.299999) (width 1) (layer "B.Cu") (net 1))
 (segment (start 90.001352 116.13001) (end 87.06999 116.13001) (width 1) (layer "B.Cu") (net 1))
 (segment (start 83.185 112.965) (end 83.185 114.013518) (width 0.8) (layer "B.Cu") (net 16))
 (segment (start 83.911492 114.74001) (end 88.73999 114.74001) (width 0.8) (layer "B.Cu") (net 16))
 (segment (start 88.73999 114.74001) (end 88.9 114.58) (width 0.8) (layer "B.Cu") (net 16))
 (segment (start 83.185 114.013518) (end 83.911492 114.74001) (width 0.8) (layer "B.Cu") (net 16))
 (segment (start 84.455 112.965) (end 85.725 112.965) (width 0.8) (layer "B.Cu") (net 15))
 (segment (start 84.455 111.916482) (end 84.455 112.965) (width 0.8) (layer "B.Cu") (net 15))
 (segment (start 83.728508 111.18999) (end 84.455 111.916482) (width 0.8) (layer "B.Cu") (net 15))
 (segment (start 81.49501 111.18999) (end 83.728508 111.18999) (width 0.8) (layer "B.Cu") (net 15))
 (segment (start 80.645 112.04) (end 81.49501 111.18999) (width 0.8) (layer "B.Cu") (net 15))
 (segment (start 84.455 106.574942) (end 83.82 105.939942) (width 0.8) (layer "B.Cu") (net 14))
 (segment (start 81.49501 109.79001) (end 83.728508 109.79001) (width 0.8) (layer "B.Cu") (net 14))
 (segment (start 84.455 109.063518) (end 84.455 108.015) (width 0.8) (layer "B.Cu") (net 14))
 (segment (start 84.455 108.015) (end 84.455 106.574942) (width 0.8) (layer "B.Cu") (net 14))
 (segment (start 83.728508 109.79001) (end 84.455 109.063518) (width 0.8) (layer "B.Cu") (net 14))
 (segment (start 80.645 108.94) (end 81.49501 109.79001) (width 0.8) (layer "B.Cu") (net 14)))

